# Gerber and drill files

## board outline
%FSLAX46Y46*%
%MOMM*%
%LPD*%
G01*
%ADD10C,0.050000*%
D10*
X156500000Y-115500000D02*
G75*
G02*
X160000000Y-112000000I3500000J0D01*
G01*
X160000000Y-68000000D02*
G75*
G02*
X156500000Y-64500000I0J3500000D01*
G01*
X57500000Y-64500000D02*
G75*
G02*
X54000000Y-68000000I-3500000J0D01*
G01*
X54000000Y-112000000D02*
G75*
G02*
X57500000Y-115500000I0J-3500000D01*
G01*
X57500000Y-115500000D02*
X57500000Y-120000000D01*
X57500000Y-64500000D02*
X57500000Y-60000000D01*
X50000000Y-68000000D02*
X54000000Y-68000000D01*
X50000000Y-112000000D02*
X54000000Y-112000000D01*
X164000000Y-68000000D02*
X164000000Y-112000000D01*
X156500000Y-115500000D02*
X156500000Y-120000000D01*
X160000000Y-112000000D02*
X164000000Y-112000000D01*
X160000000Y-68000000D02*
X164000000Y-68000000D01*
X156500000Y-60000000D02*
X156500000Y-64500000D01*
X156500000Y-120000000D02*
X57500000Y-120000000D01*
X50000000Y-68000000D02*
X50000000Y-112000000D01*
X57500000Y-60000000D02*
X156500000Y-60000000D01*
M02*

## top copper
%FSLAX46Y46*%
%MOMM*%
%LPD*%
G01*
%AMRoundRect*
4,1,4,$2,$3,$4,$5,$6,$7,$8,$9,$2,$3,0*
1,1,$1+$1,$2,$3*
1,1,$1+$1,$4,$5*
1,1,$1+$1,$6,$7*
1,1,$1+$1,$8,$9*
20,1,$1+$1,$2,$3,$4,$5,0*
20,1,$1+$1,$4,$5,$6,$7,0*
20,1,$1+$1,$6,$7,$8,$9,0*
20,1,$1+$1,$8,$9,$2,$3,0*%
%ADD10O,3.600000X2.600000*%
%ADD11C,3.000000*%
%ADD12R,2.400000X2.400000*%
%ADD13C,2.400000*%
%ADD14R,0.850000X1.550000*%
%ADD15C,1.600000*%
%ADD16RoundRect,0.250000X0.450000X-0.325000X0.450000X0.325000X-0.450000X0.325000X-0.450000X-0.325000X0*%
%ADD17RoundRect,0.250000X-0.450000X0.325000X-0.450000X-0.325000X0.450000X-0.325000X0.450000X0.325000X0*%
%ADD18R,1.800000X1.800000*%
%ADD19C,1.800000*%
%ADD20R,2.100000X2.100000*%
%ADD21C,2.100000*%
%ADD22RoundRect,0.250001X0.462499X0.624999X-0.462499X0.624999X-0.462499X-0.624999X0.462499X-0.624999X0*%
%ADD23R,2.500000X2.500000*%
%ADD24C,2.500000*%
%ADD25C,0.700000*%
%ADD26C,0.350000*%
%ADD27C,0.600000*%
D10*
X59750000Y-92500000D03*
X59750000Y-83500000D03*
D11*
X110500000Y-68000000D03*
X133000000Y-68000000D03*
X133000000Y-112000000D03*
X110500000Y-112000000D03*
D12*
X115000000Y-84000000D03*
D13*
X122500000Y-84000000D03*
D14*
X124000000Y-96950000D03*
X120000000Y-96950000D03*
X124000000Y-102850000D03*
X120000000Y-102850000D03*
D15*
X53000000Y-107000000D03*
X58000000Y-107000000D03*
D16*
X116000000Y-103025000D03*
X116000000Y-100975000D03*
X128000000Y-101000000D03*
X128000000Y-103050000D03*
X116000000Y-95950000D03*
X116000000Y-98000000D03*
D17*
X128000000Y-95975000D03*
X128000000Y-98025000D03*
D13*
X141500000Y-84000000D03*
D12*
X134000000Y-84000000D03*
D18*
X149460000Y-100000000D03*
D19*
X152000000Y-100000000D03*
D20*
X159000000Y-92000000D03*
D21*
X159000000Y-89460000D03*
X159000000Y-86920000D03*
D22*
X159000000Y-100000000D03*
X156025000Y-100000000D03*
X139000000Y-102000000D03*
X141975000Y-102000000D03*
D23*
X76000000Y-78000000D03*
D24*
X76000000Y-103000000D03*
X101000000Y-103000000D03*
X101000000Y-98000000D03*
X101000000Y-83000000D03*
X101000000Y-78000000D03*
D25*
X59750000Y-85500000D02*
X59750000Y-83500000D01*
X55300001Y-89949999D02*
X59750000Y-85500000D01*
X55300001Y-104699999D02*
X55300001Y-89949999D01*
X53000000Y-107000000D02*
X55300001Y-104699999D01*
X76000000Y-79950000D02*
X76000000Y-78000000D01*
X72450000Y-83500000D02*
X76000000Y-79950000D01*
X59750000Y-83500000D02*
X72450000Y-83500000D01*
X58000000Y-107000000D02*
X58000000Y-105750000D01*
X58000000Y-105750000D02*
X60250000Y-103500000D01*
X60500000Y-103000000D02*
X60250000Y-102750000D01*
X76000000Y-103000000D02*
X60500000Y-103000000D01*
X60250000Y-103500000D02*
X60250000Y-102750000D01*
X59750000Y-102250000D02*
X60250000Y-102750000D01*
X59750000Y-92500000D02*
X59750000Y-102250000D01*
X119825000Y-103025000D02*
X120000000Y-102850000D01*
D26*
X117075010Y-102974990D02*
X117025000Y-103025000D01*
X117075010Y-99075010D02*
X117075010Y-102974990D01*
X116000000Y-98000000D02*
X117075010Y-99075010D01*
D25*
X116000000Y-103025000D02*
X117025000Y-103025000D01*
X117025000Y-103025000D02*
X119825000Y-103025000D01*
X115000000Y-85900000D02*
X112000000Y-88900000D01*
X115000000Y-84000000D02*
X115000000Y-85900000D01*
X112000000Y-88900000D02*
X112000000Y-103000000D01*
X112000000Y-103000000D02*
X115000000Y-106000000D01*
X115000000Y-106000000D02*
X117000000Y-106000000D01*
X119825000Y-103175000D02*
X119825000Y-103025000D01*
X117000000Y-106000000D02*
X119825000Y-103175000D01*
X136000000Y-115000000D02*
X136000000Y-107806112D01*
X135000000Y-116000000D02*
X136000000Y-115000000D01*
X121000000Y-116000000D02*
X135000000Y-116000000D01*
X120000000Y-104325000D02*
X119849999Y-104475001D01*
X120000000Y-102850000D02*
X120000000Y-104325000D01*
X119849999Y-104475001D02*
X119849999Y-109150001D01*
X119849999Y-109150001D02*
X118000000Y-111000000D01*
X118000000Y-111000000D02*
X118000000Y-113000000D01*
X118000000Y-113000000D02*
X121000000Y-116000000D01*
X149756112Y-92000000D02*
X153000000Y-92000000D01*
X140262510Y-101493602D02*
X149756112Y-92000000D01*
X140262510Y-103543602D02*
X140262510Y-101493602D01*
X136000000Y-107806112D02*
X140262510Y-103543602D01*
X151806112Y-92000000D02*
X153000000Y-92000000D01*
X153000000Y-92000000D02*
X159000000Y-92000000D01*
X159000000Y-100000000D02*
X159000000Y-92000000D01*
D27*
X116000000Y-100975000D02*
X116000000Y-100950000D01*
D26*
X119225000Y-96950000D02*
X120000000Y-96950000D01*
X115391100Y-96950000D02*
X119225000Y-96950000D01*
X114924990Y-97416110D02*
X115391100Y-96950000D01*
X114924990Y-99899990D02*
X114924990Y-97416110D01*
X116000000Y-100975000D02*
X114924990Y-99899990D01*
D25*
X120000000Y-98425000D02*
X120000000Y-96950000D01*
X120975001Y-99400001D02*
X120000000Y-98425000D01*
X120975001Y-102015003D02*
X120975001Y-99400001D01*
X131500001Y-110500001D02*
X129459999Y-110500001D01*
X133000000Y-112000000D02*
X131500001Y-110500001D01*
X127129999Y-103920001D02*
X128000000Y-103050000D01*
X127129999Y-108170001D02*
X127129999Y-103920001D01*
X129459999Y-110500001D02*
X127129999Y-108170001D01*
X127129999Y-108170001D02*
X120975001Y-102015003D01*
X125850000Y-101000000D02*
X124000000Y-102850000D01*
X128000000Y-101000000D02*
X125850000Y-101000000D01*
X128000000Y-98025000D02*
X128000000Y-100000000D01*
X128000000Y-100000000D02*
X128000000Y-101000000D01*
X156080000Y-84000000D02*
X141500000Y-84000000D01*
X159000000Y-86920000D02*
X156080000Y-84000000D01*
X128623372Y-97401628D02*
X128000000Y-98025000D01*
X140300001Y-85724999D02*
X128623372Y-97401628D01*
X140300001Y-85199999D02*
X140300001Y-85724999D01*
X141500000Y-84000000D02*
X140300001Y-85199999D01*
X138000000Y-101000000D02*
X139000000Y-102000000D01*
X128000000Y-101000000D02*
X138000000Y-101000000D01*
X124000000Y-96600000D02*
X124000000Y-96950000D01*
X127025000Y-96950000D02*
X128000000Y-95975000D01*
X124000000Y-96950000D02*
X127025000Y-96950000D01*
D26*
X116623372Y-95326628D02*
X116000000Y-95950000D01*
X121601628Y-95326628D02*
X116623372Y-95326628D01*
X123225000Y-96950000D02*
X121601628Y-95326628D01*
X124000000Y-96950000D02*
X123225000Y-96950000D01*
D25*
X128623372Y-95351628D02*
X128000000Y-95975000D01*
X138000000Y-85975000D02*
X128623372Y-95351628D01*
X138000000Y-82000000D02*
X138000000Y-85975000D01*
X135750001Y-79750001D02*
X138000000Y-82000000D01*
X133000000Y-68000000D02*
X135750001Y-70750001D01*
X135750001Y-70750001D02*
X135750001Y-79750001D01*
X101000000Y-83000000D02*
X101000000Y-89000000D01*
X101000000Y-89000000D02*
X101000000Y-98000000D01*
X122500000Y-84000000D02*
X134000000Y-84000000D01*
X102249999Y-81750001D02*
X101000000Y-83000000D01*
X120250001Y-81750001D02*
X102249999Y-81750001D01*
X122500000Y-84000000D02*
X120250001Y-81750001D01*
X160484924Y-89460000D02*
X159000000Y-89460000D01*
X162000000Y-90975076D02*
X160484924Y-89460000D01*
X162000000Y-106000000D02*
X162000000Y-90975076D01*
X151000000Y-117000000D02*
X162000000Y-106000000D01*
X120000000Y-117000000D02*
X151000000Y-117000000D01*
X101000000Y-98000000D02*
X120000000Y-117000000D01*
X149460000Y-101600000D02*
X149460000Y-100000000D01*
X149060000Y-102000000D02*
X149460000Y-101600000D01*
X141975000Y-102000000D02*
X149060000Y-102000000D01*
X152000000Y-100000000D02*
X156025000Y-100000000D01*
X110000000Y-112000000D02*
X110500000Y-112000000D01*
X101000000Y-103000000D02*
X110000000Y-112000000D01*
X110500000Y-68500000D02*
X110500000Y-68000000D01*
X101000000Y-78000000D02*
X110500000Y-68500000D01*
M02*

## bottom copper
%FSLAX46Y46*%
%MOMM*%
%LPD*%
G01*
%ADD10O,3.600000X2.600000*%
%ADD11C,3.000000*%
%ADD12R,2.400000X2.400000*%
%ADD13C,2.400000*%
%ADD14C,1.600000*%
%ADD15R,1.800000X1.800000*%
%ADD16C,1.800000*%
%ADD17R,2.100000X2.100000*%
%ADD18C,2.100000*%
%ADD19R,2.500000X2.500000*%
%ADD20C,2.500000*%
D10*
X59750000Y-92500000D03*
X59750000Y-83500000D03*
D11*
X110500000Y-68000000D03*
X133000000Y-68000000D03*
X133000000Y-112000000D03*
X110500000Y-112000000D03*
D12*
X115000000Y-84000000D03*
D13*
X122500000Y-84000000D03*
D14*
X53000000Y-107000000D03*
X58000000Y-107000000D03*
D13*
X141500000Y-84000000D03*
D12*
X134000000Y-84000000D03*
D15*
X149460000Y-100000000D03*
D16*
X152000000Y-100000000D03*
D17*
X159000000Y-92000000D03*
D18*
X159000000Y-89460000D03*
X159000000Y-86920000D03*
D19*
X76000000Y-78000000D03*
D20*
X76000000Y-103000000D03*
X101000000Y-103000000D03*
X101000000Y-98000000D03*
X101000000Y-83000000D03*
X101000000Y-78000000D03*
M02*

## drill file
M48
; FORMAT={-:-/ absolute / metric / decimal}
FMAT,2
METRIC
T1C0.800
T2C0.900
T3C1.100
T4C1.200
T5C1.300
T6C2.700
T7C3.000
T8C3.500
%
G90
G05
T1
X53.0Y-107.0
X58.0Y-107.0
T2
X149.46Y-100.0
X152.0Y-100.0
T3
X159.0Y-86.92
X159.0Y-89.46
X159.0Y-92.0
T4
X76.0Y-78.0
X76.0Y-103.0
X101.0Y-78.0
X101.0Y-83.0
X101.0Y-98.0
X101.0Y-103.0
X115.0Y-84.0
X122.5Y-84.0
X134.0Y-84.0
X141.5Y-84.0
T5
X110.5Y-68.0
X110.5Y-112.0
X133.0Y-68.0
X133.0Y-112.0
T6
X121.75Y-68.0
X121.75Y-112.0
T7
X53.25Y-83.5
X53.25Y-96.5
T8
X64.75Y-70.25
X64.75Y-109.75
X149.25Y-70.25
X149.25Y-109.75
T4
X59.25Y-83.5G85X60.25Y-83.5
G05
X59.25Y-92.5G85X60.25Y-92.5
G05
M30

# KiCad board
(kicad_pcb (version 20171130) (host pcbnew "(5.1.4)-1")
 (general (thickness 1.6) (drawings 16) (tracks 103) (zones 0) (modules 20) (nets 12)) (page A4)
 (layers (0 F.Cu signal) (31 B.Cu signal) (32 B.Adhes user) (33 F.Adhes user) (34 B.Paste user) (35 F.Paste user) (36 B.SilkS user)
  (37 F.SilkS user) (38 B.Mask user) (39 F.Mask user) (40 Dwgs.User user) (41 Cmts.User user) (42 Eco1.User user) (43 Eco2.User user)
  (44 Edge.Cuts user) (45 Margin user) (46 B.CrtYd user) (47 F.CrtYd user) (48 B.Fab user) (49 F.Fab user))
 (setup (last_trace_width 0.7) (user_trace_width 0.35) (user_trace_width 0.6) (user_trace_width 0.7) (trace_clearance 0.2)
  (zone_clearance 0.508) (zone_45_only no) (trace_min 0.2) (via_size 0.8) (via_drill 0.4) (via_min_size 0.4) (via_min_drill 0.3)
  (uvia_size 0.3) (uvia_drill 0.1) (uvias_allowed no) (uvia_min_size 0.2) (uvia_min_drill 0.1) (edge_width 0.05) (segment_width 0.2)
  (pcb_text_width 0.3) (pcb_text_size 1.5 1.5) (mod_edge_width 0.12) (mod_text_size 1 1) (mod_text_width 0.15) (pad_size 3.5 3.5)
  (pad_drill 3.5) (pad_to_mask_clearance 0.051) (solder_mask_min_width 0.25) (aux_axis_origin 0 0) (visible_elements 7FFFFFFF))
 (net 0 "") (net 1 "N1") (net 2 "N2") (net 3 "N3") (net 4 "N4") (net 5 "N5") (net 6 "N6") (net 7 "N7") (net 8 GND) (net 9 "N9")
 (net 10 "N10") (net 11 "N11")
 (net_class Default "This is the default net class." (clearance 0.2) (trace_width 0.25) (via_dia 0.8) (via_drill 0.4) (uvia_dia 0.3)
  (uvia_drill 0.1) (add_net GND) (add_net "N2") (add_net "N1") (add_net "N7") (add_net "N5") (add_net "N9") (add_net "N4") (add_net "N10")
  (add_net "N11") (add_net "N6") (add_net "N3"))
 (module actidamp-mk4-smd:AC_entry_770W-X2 (layer F.Cu) (at 59.75 90 90)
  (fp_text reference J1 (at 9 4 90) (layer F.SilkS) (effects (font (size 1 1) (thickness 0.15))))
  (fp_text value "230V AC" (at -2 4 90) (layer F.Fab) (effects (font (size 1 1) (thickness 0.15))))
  (pad 1 thru_hole oval (at -2.5 0 90) (size 2.6 3.6) (drill oval 1.2 2.2) (layers *.Cu *.Mask) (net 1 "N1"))
  (pad 2 thru_hole oval (at 6.5 0 90) (size 2.6 3.6) (drill oval 1.2 2.2) (layers *.Cu *.Mask) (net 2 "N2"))
  (pad "" np_thru_hole circle (at 6.5 -6.5 90) (size 3 3) (drill 3) (layers *.Cu *.Mask))
  (pad "" np_thru_hole circle (at -6.5 -6.5 90) (size 3 3) (drill 3) (layers *.Cu *.Mask)))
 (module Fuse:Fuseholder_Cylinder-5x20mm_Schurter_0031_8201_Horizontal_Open (layer F.Cu) (at 133 68 180)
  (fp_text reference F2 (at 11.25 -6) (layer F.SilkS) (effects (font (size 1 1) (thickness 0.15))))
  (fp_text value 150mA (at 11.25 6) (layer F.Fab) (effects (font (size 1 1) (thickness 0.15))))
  (pad "" np_thru_hole circle (at 11.25 0 180) (size 2.7 2.7) (drill 2.7) (layers *.Cu *.Mask))
  (pad 2 thru_hole circle (at 22.5 0 180) (size 3 3) (drill 1.3) (layers *.Cu *.Mask) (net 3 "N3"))
  (pad 1 thru_hole circle (at 0 0 180) (size 3 3) (drill 1.3) (layers *.Cu *.Mask) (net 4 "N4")))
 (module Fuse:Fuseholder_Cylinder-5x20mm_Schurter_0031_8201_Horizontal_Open (layer F.Cu) (at 133 112 180)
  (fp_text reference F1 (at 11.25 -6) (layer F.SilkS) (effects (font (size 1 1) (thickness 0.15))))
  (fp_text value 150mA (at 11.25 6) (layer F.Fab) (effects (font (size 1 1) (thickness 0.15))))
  (pad 1 thru_hole circle (at 0 0 180) (size 3 3) (drill 1.3) (layers *.Cu *.Mask) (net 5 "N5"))
  (pad 2 thru_hole circle (at 22.5 0 180) (size 3 3) (drill 1.3) (layers *.Cu *.Mask) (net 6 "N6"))
  (pad "" np_thru_hole circle (at 11.25 0 180) (size 2.7 2.7) (drill 2.7) (layers *.Cu *.Mask)))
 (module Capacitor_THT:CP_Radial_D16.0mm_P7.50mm (layer F.Cu) (at 115 84)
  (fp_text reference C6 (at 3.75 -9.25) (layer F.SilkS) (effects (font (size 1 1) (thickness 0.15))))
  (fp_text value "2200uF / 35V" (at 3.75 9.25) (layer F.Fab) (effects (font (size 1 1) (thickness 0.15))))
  (pad 1 thru_hole rect (at 0 0) (size 2.4 2.4) (drill 1.2) (layers *.Cu *.Mask) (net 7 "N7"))
  (pad 2 thru_hole circle (at 7.5 0) (size 2.4 2.4) (drill 1.2) (layers *.Cu *.Mask) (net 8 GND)))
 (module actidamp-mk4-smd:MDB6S (layer F.Cu) (at 122 100)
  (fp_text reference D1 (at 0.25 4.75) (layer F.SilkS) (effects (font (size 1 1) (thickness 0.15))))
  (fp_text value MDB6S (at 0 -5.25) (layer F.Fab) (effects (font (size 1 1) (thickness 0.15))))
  (pad 4 smd rect (at 2 -3.05) (size 0.85 1.55) (layers F.Cu F.Paste F.Mask) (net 4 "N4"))
  (pad 3 smd rect (at -2 -3.05) (size 0.85 1.55) (layers F.Cu F.Paste F.Mask) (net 5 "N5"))
  (pad 2 smd rect (at 2 2.85) (size 0.85 1.55) (layers F.Cu F.Paste F.Mask) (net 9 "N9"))
  (pad 1 smd rect (at -2 2.85) (size 0.85 1.55) (layers F.Cu F.Paste F.Mask) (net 7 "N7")))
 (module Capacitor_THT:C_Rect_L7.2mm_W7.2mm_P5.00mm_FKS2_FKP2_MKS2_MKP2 (layer F.Cu) (at 53 107)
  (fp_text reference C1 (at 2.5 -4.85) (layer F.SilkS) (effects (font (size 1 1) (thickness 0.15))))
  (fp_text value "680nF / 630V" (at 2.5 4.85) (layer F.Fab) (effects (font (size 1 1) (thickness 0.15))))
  (pad 1 thru_hole circle (at 0 0) (size 1.6 1.6) (drill 0.8) (layers *.Cu *.Mask) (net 2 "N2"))
  (pad 2 thru_hole circle (at 5 0) (size 1.6 1.6) (drill 0.8) (layers *.Cu *.Mask) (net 1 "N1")))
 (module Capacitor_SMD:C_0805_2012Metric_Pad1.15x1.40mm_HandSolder (layer F.Cu) (at 116 102 90)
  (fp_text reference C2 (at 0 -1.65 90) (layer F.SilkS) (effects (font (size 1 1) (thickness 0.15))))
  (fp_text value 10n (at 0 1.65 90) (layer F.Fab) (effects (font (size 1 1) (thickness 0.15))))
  (pad 1 smd roundrect (at -1.025 0 90) (size 1.15 1.4) (layers F.Cu F.Paste F.Mask) (roundrect_rratio 0.217391) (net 7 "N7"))
  (pad 2 smd roundrect (at 1.025 0 90) (size 1.15 1.4) (layers F.Cu F.Paste F.Mask) (roundrect_rratio 0.217391) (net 5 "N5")))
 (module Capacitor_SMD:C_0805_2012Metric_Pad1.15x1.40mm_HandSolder (layer F.Cu) (at 128 102.025 90)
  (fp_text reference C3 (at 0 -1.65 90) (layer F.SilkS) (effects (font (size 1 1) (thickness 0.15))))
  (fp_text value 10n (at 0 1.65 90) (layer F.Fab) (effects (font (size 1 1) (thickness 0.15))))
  (pad 2 smd roundrect (at 1.025 0 90) (size 1.15 1.4) (layers F.Cu F.Paste F.Mask) (roundrect_rratio 0.217391) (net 9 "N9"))
  (pad 1 smd roundrect (at -1.025 0 90) (size 1.15 1.4) (layers F.Cu F.Paste F.Mask) (roundrect_rratio 0.217391) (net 5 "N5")))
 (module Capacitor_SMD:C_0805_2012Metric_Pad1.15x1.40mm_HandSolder (layer F.Cu) (at 116 96.975 90)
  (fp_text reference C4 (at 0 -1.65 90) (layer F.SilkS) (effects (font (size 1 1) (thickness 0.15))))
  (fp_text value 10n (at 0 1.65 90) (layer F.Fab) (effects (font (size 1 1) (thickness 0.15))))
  (pad 2 smd roundrect (at 1.025 0 90) (size 1.15 1.4) (layers F.Cu F.Paste F.Mask) (roundrect_rratio 0.217391) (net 4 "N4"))
  (pad 1 smd roundrect (at -1.025 0 90) (size 1.15 1.4) (layers F.Cu F.Paste F.Mask) (roundrect_rratio 0.217391) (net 7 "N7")))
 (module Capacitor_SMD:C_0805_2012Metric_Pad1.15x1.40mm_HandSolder (layer F.Cu) (at 128 97 270)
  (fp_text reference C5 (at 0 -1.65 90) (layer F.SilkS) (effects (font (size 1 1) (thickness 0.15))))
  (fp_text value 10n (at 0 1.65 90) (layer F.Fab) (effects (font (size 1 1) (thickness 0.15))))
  (pad 1 smd roundrect (at -1.025 0 270) (size 1.15 1.4) (layers F.Cu F.Paste F.Mask) (roundrect_rratio 0.217391) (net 4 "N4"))
  (pad 2 smd roundrect (at 1.025 0 270) (size 1.15 1.4) (layers F.Cu F.Paste F.Mask) (roundrect_rratio 0.217391) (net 9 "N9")))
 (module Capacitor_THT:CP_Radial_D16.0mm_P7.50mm (layer F.Cu) (at 134 84)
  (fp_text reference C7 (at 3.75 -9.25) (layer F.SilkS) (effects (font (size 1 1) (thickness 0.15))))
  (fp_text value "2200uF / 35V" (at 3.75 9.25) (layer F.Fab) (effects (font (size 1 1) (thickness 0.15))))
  (pad 2 thru_hole circle (at 7.5 0) (size 2.4 2.4) (drill 1.2) (layers *.Cu *.Mask) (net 9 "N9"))
  (pad 1 thru_hole rect (at 0 0) (size 2.4 2.4) (drill 1.2) (layers *.Cu *.Mask) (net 8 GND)))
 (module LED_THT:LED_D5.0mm (layer F.Cu) (at 149.46 100)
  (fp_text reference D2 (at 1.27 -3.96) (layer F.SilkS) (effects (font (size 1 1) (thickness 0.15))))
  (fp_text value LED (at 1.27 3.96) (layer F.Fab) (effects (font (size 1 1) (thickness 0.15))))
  (pad 1 thru_hole rect (at 0 0) (size 1.8 1.8) (drill 0.9) (layers *.Cu *.Mask) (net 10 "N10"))
  (pad 2 thru_hole circle (at 2.54 0) (size 1.8 1.8) (drill 0.9) (layers *.Cu *.Mask) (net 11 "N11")))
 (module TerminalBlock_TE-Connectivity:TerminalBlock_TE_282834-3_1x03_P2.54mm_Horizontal (layer F.Cu) (at 159 92 90)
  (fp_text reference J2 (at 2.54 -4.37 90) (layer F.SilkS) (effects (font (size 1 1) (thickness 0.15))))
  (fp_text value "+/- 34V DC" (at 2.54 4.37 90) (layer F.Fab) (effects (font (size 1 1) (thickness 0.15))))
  (pad 1 thru_hole rect (at 0 0 90) (size 2.1 2.1) (drill 1.1) (layers *.Cu *.Mask) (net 7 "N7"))
  (pad 2 thru_hole circle (at 2.54 0 90) (size 2.1 2.1) (drill 1.1) (layers *.Cu *.Mask) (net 8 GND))
  (pad 3 thru_hole circle (at 5.08 0 90) (size 2.1 2.1) (drill 1.1) (layers *.Cu *.Mask) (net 9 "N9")))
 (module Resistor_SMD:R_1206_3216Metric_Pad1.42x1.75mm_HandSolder (layer F.Cu) (at 157.5125 100 180)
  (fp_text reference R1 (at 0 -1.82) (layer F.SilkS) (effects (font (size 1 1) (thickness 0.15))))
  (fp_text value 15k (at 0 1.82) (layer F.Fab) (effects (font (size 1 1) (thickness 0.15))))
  (pad 1 smd roundrect (at -1.4875 0 180) (size 1.425 1.75) (layers F.Cu F.Paste F.Mask) (roundrect_rratio 0.175439) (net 7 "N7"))
  (pad 2 smd roundrect (at 1.4875 0 180) (size 1.425 1.75) (layers F.Cu F.Paste F.Mask) (roundrect_rratio 0.175439) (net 11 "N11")))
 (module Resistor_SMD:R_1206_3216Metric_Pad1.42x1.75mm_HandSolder (layer F.Cu) (at 140.4875 102 180)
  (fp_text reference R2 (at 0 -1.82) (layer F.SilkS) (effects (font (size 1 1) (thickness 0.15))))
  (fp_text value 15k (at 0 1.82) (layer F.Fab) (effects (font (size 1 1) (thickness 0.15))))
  (pad 2 smd roundrect (at 1.4875 0 180) (size 1.425 1.75) (layers F.Cu F.Paste F.Mask) (roundrect_rratio 0.175439) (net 9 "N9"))
  (pad 1 smd roundrect (at -1.4875 0 180) (size 1.425 1.75) (layers F.Cu F.Paste F.Mask) (roundrect_rratio 0.175439) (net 10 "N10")))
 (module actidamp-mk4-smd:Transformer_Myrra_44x (layer F.Cu) (at 76 78)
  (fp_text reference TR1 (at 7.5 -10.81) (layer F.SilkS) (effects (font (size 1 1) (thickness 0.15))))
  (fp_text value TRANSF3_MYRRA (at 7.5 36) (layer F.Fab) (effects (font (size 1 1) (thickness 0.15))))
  (pad 1 thru_hole rect (at 0 0) (size 2.5 2.5) (drill 1.2) (layers *.Cu *.Mask) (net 2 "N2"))
  (pad 5 thru_hole circle (at 0 25) (size 2.5 2.5) (drill 1.2) (layers *.Cu *.Mask) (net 1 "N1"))
  (pad 6 thru_hole circle (at 25 25) (size 2.5 2.5) (drill 1.2) (layers *.Cu *.Mask) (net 6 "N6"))
  (pad 7 thru_hole circle (at 25 20) (size 2.5 2.5) (drill 1.2) (layers *.Cu *.Mask) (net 8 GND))
  (pad 9 thru_hole circle (at 25 5) (size 2.5 2.5) (drill 1.2) (layers *.Cu *.Mask) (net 8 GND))
  (pad 10 thru_hole circle (at 25 0) (size 2.5 2.5) (drill 1.2) (layers *.Cu *.Mask) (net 3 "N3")))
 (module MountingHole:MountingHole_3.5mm (layer F.Cu) (at 64.75 109.75)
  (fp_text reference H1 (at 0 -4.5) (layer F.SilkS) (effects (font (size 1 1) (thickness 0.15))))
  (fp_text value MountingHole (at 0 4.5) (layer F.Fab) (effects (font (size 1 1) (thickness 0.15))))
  (pad 1 np_thru_hole circle (at 0 0) (size 3.5 3.5) (drill 3.5) (layers *.Cu *.Mask)))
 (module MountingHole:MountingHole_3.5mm (layer F.Cu) (at 64.75 70.25)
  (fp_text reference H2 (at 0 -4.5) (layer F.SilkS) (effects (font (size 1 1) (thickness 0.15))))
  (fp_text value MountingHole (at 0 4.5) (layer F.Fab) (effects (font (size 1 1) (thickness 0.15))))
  (pad 1 np_thru_hole circle (at 0 0) (size 3.5 3.5) (drill 3.5) (layers *.Cu *.Mask)))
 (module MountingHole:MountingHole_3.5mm (layer F.Cu) (at 149.25 109.75)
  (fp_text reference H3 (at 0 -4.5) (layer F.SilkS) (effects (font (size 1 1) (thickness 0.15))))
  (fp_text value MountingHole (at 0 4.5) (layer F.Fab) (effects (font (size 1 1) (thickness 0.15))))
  (pad 1 np_thru_hole circle (at 0 0) (size 3.5 3.5) (drill 3.5) (layers *.Cu *.Mask)))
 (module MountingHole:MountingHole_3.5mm (layer F.Cu) (at 149.25 70.25)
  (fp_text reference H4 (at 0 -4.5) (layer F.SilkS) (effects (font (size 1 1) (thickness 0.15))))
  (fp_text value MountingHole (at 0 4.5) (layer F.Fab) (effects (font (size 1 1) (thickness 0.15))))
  (pad 1 np_thru_hole circle (at 0 0) (size 3.5 3.5) (drill 3.5) (layers *.Cu *.Mask)))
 (gr_arc (start 160 115.5) (end 160 112) (angle -90) (layer Edge.Cuts) (width 0.05))
 (gr_arc (start 160 64.5) (end 156.5 64.5) (angle -90) (layer Edge.Cuts) (width 0.05))
 (gr_arc (start 54 64.5) (end 54 68) (angle -90) (layer Edge.Cuts) (width 0.05))
 (gr_arc (start 54 115.5) (end 57.5 115.5) (angle -90) (layer Edge.Cuts) (width 0.05))
 (gr_line (start 57.5 115.5) (end 57.5 120) (layer Edge.Cuts) (width 0.05))
 (gr_line (start 57.5 64.5) (end 57.5 60) (layer Edge.Cuts) (width 0.05))
 (gr_line (start 50 68) (end 54 68) (layer Edge.Cuts) (width 0.05))
 (gr_line (start 50 112) (end 54 112) (layer Edge.Cuts) (width 0.05))
 (gr_line (start 164 68) (end 164 112) (layer Edge.Cuts) (width 0.05))
 (gr_line (start 156.5 115.5) (end 156.5 120) (layer Edge.Cuts) (width 0.05))
 (gr_line (start 160 112) (end 164 112) (layer Edge.Cuts) (width 0.05))
 (gr_line (start 160 68) (end 164 68) (layer Edge.Cuts) (width 0.05))
 (gr_line (start 156.5 60) (end 156.5 64.5) (layer Edge.Cuts) (width 0.05))
 (gr_line (start 156.5 120) (end 57.5 120) (layer Edge.Cuts) (width 0.05))
 (gr_line (start 50 68) (end 50 112) (layer Edge.Cuts) (width 0.05))
 (gr_line (start 57.5 60) (end 156.5 60) (layer Edge.Cuts) (width 0.05))
 (segment (start 59.75 85.5) (end 59.75 83.5) (width 0.7) (layer F.Cu) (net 2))
 (segment (start 55.300001 89.949999) (end 59.75 85.5) (width 0.7) (layer F.Cu) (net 2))
 (segment (start 55.300001 104.699999) (end 55.300001 89.949999) (width 0.7) (layer F.Cu) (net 2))
 (segment (start 53 107) (end 55.300001 104.699999) (width 0.7) (layer F.Cu) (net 2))
 (segment (start 76 79.95) (end 76 78) (width 0.7) (layer F.Cu) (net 2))
 (segment (start 72.45 83.5) (end 76 79.95) (width 0.7) (layer F.Cu) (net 2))
 (segment (start 59.75 83.5) (end 72.45 83.5) (width 0.7) (layer F.Cu) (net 2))
 (segment (start 58 107) (end 58 105.75) (width 0.7) (layer F.Cu) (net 1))
 (segment (start 58 105.75) (end 60.25 103.5) (width 0.7) (layer F.Cu) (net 1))
 (segment (start 60.5 103) (end 60.25 102.75) (width 0.7) (layer F.Cu) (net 1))
 (segment (start 76 103) (end 60.5 103) (width 0.7) (layer F.Cu) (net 1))
 (segment (start 60.25 103.5) (end 60.25 102.75) (width 0.7) (layer F.Cu) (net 1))
 (segment (start 59.75 102.25) (end 60.25 102.75) (width 0.7) (layer F.Cu) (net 1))
 (segment (start 59.75 92.5) (end 59.75 102.25) (width 0.7) (layer F.Cu) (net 1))
 (segment (start 119.825 103.025) (end 120 102.85) (width 0.7) (layer F.Cu) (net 7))
 (segment (start 117.07501 102.97499) (end 117.025 103.025) (width 0.35) (layer F.Cu) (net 7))
 (segment (start 117.07501 99.07501) (end 117.07501 102.97499) (width 0.35) (layer F.Cu) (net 7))
 (segment (start 116 98) (end 117.07501 99.07501) (width 0.35) (layer F.Cu) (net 7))
 (segment (start 116 103.025) (end 117.025 103.025) (width 0.7) (layer F.Cu) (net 7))
 (segment (start 117.025 103.025) (end 119.825 103.025) (width 0.7) (layer F.Cu) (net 7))
 (segment (start 115 85.9) (end 112 88.9) (width 0.7) (layer F.Cu) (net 7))
 (segment (start 115 84) (end 115 85.9) (width 0.7) (layer F.Cu) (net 7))
 (segment (start 112 88.9) (end 112 103) (width 0.7) (layer F.Cu) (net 7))
 (segment (start 112 103) (end 115 106) (width 0.7) (layer F.Cu) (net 7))
 (segment (start 115 106) (end 117 106) (width 0.7) (layer F.Cu) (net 7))
 (segment (start 119.825 103.175) (end 119.825 103.025) (width 0.7) (layer F.Cu) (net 7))
 (segment (start 117 106) (end 119.825 103.175) (width 0.7) (layer F.Cu) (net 7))
 (segment (start 136 115) (end 136 107.806112) (width 0.7) (layer F.Cu) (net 7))
 (segment (start 135 116) (end 136 115) (width 0.7) (layer F.Cu) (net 7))
 (segment (start 121 116) (end 135 116) (width 0.7) (layer F.Cu) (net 7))
 (segment (start 120 104.325) (end 119.849999 104.475001) (width 0.7) (layer F.Cu) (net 7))
 (segment (start 120 102.85) (end 120 104.325) (width 0.7) (layer F.Cu) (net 7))
 (segment (start 119.849999 104.475001) (end 119.849999 109.150001) (width 0.7) (layer F.Cu) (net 7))
 (segment (start 119.849999 109.150001) (end 118 111) (width 0.7) (layer F.Cu) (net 7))
 (segment (start 118 111) (end 118 113) (width 0.7) (layer F.Cu) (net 7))
 (segment (start 118 113) (end 121 116) (width 0.7) (layer F.Cu) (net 7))
 (segment (start 149.756112 92) (end 153 92) (width 0.7) (layer F.Cu) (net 7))
 (segment (start 140.26251 101.493602) (end 149.756112 92) (width 0.7) (layer F.Cu) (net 7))
 (segment (start 140.26251 103.543602) (end 140.26251 101.493602) (width 0.7) (layer F.Cu) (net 7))
 (segment (start 136 107.806112) (end 140.26251 103.543602) (width 0.7) (layer F.Cu) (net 7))
 (segment (start 151.806112 92) (end 153 92) (width 0.7) (layer F.Cu) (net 7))
 (segment (start 153 92) (end 159 92) (width 0.7) (layer F.Cu) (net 7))
 (segment (start 159 100) (end 159 92) (width 0.7) (layer F.Cu) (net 7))
 (segment (start 116 100.975) (end 116 100.95) (width 0.6) (layer F.Cu) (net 5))
 (segment (start 119.225 96.95) (end 120 96.95) (width 0.35) (layer F.Cu) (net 5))
 (segment (start 115.3911 96.95) (end 119.225 96.95) (width 0.35) (layer F.Cu) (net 5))
 (segment (start 114.92499 97.41611) (end 115.3911 96.95) (width 0.35) (layer F.Cu) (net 5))
 (segment (start 114.92499 99.89999) (end 114.92499 97.41611) (width 0.35) (layer F.Cu) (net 5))
 (segment (start 116 100.975) (end 114.92499 99.89999) (width 0.35) (layer F.Cu) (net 5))
 (segment (start 120 98.425) (end 120 96.95) (width 0.7) (layer F.Cu) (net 5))
 (segment (start 120.975001 99.400001) (end 120 98.425) (width 0.7) (layer F.Cu) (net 5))
 (segment (start 120.975001 102.015003) (end 120.975001 99.400001) (width 0.7) (layer F.Cu) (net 5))
 (segment (start 131.500001 110.500001) (end 129.459999 110.500001) (width 0.7) (layer F.Cu) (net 5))
 (segment (start 133 112) (end 131.500001 110.500001) (width 0.7) (layer F.Cu) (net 5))
 (segment (start 127.129999 103.920001) (end 128 103.05) (width 0.7) (layer F.Cu) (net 5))
 (segment (start 127.129999 108.170001) (end 127.129999 103.920001) (width 0.7) (layer F.Cu) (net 5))
 (segment (start 129.459999 110.500001) (end 127.129999 108.170001) (width 0.7) (layer F.Cu) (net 5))
 (segment (start 127.129999 108.170001) (end 120.975001 102.015003) (width 0.7) (layer F.Cu) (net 5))
 (segment (start 125.85 101) (end 124 102.85) (width 0.7) (layer F.Cu) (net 9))
 (segment (start 128 101) (end 125.85 101) (width 0.7) (layer F.Cu) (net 9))
 (segment (start 128 98.025) (end 128 100) (width 0.7) (layer F.Cu) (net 9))
 (segment (start 128 100) (end 128 101) (width 0.7) (layer F.Cu) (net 9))
 (segment (start 156.08 84) (end 141.5 84) (width 0.7) (layer F.Cu) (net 9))
 (segment (start 159 86.92) (end 156.08 84) (width 0.7) (layer F.Cu) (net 9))
 (segment (start 128.623372 97.401628) (end 128 98.025) (width 0.7) (layer F.Cu) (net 9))
 (segment (start 140.300001 85.724999) (end 128.623372 97.401628) (width 0.7) (layer F.Cu) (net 9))
 (segment (start 140.300001 85.199999) (end 140.300001 85.724999) (width 0.7) (layer F.Cu) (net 9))
 (segment (start 141.5 84) (end 140.300001 85.199999) (width 0.7) (layer F.Cu) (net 9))
 (segment (start 138 101) (end 139 102) (width 0.7) (layer F.Cu) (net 9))
 (segment (start 128 101) (end 138 101) (width 0.7) (layer F.Cu) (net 9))
 (segment (start 124 96.6) (end 124 96.95) (width 0.7) (layer F.Cu) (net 4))
 (segment (start 127.025 96.95) (end 128 95.975) (width 0.7) (layer F.Cu) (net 4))
 (segment (start 124 96.95) (end 127.025 96.95) (width 0.7) (layer F.Cu) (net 4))
 (segment (start 116.623372 95.326628) (end 116 95.95) (width 0.35) (layer F.Cu) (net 4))
 (segment (start 121.601628 95.326628) (end 116.623372 95.326628) (width 0.35) (layer F.Cu) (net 4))
 (segment (start 123.225 96.95) (end 121.601628 95.326628) (width 0.35) (layer F.Cu) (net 4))
 (segment (start 124 96.95) (end 123.225 96.95) (width 0.35) (layer F.Cu) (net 4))
 (segment (start 128.623372 95.351628) (end 128 95.975) (width 0.7) (layer F.Cu) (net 4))
 (segment (start 138 85.975) (end 128.623372 95.351628) (width 0.7) (layer F.Cu) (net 4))
 (segment (start 138 82) (end 138 85.975) (width 0.7) (layer F.Cu) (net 4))
 (segment (start 135.750001 79.750001) (end 138 82) (width 0.7) (layer F.Cu) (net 4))
 (segment (start 133 68) (end 135.750001 70.750001) (width 0.7) (layer F.Cu) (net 4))
 (segment (start 135.750001 70.750001) (end 135.750001 79.750001) (width 0.7) (layer F.Cu) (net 4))
 (segment (start 101 83) (end 101 89) (width 0.7) (layer F.Cu) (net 8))
 (segment (start 101 89) (end 101 98) (width 0.7) (layer F.Cu) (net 8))
 (segment (start 122.5 84) (end 134 84) (width 0.7) (layer F.Cu) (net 8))
 (segment (start 102.249999 81.750001) (end 101 83) (width 0.7) (layer F.Cu) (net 8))
 (segment (start 120.250001 81.750001) (end 102.249999 81.750001) (width 0.7) (layer F.Cu) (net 8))
 (segment (start 122.5 84) (end 120.250001 81.750001) (width 0.7) (layer F.Cu) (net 8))
 (segment (start 160.484924 89.46) (end 159 89.46) (width 0.7) (layer F.Cu) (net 8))
 (segment (start 162 90.975076) (end 160.484924 89.46) (width 0.7) (layer F.Cu) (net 8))
 (segment (start 162 106) (end 162 90.975076) (width 0.7) (layer F.Cu) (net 8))
 (segment (start 151 117) (end 162 106) (width 0.7) (layer F.Cu) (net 8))
 (segment (start 120 117) (end 151 117) (width 0.7) (layer F.Cu) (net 8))
 (segment (start 101 98) (end 120 117) (width 0.7) (layer F.Cu) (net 8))
 (segment (start 149.46 101.6) (end 149.46 100) (width 0.7) (layer F.Cu) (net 10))
 (segment (start 149.06 102) (end 149.46 101.6) (width 0.7) (layer F.Cu) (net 10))
 (segment (start 141.975 102) (end 149.06 102) (width 0.7) (layer F.Cu) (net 10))
 (segment (start 152 100) (end 156.025 100) (width 0.7) (layer F.Cu) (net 11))
 (segment (start 110 112) (end 110.5 112) (width 0.7) (layer F.Cu) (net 6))
 (segment (start 101 103) (end 110 112) (width 0.7) (layer F.Cu) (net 6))
 (segment (start 110.5 68.5) (end 110.5 68) (width 0.7) (layer F.Cu) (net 3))
 (segment (start 101 78) (end 110.5 68.5) (width 0.7) (layer F.Cu) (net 3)))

